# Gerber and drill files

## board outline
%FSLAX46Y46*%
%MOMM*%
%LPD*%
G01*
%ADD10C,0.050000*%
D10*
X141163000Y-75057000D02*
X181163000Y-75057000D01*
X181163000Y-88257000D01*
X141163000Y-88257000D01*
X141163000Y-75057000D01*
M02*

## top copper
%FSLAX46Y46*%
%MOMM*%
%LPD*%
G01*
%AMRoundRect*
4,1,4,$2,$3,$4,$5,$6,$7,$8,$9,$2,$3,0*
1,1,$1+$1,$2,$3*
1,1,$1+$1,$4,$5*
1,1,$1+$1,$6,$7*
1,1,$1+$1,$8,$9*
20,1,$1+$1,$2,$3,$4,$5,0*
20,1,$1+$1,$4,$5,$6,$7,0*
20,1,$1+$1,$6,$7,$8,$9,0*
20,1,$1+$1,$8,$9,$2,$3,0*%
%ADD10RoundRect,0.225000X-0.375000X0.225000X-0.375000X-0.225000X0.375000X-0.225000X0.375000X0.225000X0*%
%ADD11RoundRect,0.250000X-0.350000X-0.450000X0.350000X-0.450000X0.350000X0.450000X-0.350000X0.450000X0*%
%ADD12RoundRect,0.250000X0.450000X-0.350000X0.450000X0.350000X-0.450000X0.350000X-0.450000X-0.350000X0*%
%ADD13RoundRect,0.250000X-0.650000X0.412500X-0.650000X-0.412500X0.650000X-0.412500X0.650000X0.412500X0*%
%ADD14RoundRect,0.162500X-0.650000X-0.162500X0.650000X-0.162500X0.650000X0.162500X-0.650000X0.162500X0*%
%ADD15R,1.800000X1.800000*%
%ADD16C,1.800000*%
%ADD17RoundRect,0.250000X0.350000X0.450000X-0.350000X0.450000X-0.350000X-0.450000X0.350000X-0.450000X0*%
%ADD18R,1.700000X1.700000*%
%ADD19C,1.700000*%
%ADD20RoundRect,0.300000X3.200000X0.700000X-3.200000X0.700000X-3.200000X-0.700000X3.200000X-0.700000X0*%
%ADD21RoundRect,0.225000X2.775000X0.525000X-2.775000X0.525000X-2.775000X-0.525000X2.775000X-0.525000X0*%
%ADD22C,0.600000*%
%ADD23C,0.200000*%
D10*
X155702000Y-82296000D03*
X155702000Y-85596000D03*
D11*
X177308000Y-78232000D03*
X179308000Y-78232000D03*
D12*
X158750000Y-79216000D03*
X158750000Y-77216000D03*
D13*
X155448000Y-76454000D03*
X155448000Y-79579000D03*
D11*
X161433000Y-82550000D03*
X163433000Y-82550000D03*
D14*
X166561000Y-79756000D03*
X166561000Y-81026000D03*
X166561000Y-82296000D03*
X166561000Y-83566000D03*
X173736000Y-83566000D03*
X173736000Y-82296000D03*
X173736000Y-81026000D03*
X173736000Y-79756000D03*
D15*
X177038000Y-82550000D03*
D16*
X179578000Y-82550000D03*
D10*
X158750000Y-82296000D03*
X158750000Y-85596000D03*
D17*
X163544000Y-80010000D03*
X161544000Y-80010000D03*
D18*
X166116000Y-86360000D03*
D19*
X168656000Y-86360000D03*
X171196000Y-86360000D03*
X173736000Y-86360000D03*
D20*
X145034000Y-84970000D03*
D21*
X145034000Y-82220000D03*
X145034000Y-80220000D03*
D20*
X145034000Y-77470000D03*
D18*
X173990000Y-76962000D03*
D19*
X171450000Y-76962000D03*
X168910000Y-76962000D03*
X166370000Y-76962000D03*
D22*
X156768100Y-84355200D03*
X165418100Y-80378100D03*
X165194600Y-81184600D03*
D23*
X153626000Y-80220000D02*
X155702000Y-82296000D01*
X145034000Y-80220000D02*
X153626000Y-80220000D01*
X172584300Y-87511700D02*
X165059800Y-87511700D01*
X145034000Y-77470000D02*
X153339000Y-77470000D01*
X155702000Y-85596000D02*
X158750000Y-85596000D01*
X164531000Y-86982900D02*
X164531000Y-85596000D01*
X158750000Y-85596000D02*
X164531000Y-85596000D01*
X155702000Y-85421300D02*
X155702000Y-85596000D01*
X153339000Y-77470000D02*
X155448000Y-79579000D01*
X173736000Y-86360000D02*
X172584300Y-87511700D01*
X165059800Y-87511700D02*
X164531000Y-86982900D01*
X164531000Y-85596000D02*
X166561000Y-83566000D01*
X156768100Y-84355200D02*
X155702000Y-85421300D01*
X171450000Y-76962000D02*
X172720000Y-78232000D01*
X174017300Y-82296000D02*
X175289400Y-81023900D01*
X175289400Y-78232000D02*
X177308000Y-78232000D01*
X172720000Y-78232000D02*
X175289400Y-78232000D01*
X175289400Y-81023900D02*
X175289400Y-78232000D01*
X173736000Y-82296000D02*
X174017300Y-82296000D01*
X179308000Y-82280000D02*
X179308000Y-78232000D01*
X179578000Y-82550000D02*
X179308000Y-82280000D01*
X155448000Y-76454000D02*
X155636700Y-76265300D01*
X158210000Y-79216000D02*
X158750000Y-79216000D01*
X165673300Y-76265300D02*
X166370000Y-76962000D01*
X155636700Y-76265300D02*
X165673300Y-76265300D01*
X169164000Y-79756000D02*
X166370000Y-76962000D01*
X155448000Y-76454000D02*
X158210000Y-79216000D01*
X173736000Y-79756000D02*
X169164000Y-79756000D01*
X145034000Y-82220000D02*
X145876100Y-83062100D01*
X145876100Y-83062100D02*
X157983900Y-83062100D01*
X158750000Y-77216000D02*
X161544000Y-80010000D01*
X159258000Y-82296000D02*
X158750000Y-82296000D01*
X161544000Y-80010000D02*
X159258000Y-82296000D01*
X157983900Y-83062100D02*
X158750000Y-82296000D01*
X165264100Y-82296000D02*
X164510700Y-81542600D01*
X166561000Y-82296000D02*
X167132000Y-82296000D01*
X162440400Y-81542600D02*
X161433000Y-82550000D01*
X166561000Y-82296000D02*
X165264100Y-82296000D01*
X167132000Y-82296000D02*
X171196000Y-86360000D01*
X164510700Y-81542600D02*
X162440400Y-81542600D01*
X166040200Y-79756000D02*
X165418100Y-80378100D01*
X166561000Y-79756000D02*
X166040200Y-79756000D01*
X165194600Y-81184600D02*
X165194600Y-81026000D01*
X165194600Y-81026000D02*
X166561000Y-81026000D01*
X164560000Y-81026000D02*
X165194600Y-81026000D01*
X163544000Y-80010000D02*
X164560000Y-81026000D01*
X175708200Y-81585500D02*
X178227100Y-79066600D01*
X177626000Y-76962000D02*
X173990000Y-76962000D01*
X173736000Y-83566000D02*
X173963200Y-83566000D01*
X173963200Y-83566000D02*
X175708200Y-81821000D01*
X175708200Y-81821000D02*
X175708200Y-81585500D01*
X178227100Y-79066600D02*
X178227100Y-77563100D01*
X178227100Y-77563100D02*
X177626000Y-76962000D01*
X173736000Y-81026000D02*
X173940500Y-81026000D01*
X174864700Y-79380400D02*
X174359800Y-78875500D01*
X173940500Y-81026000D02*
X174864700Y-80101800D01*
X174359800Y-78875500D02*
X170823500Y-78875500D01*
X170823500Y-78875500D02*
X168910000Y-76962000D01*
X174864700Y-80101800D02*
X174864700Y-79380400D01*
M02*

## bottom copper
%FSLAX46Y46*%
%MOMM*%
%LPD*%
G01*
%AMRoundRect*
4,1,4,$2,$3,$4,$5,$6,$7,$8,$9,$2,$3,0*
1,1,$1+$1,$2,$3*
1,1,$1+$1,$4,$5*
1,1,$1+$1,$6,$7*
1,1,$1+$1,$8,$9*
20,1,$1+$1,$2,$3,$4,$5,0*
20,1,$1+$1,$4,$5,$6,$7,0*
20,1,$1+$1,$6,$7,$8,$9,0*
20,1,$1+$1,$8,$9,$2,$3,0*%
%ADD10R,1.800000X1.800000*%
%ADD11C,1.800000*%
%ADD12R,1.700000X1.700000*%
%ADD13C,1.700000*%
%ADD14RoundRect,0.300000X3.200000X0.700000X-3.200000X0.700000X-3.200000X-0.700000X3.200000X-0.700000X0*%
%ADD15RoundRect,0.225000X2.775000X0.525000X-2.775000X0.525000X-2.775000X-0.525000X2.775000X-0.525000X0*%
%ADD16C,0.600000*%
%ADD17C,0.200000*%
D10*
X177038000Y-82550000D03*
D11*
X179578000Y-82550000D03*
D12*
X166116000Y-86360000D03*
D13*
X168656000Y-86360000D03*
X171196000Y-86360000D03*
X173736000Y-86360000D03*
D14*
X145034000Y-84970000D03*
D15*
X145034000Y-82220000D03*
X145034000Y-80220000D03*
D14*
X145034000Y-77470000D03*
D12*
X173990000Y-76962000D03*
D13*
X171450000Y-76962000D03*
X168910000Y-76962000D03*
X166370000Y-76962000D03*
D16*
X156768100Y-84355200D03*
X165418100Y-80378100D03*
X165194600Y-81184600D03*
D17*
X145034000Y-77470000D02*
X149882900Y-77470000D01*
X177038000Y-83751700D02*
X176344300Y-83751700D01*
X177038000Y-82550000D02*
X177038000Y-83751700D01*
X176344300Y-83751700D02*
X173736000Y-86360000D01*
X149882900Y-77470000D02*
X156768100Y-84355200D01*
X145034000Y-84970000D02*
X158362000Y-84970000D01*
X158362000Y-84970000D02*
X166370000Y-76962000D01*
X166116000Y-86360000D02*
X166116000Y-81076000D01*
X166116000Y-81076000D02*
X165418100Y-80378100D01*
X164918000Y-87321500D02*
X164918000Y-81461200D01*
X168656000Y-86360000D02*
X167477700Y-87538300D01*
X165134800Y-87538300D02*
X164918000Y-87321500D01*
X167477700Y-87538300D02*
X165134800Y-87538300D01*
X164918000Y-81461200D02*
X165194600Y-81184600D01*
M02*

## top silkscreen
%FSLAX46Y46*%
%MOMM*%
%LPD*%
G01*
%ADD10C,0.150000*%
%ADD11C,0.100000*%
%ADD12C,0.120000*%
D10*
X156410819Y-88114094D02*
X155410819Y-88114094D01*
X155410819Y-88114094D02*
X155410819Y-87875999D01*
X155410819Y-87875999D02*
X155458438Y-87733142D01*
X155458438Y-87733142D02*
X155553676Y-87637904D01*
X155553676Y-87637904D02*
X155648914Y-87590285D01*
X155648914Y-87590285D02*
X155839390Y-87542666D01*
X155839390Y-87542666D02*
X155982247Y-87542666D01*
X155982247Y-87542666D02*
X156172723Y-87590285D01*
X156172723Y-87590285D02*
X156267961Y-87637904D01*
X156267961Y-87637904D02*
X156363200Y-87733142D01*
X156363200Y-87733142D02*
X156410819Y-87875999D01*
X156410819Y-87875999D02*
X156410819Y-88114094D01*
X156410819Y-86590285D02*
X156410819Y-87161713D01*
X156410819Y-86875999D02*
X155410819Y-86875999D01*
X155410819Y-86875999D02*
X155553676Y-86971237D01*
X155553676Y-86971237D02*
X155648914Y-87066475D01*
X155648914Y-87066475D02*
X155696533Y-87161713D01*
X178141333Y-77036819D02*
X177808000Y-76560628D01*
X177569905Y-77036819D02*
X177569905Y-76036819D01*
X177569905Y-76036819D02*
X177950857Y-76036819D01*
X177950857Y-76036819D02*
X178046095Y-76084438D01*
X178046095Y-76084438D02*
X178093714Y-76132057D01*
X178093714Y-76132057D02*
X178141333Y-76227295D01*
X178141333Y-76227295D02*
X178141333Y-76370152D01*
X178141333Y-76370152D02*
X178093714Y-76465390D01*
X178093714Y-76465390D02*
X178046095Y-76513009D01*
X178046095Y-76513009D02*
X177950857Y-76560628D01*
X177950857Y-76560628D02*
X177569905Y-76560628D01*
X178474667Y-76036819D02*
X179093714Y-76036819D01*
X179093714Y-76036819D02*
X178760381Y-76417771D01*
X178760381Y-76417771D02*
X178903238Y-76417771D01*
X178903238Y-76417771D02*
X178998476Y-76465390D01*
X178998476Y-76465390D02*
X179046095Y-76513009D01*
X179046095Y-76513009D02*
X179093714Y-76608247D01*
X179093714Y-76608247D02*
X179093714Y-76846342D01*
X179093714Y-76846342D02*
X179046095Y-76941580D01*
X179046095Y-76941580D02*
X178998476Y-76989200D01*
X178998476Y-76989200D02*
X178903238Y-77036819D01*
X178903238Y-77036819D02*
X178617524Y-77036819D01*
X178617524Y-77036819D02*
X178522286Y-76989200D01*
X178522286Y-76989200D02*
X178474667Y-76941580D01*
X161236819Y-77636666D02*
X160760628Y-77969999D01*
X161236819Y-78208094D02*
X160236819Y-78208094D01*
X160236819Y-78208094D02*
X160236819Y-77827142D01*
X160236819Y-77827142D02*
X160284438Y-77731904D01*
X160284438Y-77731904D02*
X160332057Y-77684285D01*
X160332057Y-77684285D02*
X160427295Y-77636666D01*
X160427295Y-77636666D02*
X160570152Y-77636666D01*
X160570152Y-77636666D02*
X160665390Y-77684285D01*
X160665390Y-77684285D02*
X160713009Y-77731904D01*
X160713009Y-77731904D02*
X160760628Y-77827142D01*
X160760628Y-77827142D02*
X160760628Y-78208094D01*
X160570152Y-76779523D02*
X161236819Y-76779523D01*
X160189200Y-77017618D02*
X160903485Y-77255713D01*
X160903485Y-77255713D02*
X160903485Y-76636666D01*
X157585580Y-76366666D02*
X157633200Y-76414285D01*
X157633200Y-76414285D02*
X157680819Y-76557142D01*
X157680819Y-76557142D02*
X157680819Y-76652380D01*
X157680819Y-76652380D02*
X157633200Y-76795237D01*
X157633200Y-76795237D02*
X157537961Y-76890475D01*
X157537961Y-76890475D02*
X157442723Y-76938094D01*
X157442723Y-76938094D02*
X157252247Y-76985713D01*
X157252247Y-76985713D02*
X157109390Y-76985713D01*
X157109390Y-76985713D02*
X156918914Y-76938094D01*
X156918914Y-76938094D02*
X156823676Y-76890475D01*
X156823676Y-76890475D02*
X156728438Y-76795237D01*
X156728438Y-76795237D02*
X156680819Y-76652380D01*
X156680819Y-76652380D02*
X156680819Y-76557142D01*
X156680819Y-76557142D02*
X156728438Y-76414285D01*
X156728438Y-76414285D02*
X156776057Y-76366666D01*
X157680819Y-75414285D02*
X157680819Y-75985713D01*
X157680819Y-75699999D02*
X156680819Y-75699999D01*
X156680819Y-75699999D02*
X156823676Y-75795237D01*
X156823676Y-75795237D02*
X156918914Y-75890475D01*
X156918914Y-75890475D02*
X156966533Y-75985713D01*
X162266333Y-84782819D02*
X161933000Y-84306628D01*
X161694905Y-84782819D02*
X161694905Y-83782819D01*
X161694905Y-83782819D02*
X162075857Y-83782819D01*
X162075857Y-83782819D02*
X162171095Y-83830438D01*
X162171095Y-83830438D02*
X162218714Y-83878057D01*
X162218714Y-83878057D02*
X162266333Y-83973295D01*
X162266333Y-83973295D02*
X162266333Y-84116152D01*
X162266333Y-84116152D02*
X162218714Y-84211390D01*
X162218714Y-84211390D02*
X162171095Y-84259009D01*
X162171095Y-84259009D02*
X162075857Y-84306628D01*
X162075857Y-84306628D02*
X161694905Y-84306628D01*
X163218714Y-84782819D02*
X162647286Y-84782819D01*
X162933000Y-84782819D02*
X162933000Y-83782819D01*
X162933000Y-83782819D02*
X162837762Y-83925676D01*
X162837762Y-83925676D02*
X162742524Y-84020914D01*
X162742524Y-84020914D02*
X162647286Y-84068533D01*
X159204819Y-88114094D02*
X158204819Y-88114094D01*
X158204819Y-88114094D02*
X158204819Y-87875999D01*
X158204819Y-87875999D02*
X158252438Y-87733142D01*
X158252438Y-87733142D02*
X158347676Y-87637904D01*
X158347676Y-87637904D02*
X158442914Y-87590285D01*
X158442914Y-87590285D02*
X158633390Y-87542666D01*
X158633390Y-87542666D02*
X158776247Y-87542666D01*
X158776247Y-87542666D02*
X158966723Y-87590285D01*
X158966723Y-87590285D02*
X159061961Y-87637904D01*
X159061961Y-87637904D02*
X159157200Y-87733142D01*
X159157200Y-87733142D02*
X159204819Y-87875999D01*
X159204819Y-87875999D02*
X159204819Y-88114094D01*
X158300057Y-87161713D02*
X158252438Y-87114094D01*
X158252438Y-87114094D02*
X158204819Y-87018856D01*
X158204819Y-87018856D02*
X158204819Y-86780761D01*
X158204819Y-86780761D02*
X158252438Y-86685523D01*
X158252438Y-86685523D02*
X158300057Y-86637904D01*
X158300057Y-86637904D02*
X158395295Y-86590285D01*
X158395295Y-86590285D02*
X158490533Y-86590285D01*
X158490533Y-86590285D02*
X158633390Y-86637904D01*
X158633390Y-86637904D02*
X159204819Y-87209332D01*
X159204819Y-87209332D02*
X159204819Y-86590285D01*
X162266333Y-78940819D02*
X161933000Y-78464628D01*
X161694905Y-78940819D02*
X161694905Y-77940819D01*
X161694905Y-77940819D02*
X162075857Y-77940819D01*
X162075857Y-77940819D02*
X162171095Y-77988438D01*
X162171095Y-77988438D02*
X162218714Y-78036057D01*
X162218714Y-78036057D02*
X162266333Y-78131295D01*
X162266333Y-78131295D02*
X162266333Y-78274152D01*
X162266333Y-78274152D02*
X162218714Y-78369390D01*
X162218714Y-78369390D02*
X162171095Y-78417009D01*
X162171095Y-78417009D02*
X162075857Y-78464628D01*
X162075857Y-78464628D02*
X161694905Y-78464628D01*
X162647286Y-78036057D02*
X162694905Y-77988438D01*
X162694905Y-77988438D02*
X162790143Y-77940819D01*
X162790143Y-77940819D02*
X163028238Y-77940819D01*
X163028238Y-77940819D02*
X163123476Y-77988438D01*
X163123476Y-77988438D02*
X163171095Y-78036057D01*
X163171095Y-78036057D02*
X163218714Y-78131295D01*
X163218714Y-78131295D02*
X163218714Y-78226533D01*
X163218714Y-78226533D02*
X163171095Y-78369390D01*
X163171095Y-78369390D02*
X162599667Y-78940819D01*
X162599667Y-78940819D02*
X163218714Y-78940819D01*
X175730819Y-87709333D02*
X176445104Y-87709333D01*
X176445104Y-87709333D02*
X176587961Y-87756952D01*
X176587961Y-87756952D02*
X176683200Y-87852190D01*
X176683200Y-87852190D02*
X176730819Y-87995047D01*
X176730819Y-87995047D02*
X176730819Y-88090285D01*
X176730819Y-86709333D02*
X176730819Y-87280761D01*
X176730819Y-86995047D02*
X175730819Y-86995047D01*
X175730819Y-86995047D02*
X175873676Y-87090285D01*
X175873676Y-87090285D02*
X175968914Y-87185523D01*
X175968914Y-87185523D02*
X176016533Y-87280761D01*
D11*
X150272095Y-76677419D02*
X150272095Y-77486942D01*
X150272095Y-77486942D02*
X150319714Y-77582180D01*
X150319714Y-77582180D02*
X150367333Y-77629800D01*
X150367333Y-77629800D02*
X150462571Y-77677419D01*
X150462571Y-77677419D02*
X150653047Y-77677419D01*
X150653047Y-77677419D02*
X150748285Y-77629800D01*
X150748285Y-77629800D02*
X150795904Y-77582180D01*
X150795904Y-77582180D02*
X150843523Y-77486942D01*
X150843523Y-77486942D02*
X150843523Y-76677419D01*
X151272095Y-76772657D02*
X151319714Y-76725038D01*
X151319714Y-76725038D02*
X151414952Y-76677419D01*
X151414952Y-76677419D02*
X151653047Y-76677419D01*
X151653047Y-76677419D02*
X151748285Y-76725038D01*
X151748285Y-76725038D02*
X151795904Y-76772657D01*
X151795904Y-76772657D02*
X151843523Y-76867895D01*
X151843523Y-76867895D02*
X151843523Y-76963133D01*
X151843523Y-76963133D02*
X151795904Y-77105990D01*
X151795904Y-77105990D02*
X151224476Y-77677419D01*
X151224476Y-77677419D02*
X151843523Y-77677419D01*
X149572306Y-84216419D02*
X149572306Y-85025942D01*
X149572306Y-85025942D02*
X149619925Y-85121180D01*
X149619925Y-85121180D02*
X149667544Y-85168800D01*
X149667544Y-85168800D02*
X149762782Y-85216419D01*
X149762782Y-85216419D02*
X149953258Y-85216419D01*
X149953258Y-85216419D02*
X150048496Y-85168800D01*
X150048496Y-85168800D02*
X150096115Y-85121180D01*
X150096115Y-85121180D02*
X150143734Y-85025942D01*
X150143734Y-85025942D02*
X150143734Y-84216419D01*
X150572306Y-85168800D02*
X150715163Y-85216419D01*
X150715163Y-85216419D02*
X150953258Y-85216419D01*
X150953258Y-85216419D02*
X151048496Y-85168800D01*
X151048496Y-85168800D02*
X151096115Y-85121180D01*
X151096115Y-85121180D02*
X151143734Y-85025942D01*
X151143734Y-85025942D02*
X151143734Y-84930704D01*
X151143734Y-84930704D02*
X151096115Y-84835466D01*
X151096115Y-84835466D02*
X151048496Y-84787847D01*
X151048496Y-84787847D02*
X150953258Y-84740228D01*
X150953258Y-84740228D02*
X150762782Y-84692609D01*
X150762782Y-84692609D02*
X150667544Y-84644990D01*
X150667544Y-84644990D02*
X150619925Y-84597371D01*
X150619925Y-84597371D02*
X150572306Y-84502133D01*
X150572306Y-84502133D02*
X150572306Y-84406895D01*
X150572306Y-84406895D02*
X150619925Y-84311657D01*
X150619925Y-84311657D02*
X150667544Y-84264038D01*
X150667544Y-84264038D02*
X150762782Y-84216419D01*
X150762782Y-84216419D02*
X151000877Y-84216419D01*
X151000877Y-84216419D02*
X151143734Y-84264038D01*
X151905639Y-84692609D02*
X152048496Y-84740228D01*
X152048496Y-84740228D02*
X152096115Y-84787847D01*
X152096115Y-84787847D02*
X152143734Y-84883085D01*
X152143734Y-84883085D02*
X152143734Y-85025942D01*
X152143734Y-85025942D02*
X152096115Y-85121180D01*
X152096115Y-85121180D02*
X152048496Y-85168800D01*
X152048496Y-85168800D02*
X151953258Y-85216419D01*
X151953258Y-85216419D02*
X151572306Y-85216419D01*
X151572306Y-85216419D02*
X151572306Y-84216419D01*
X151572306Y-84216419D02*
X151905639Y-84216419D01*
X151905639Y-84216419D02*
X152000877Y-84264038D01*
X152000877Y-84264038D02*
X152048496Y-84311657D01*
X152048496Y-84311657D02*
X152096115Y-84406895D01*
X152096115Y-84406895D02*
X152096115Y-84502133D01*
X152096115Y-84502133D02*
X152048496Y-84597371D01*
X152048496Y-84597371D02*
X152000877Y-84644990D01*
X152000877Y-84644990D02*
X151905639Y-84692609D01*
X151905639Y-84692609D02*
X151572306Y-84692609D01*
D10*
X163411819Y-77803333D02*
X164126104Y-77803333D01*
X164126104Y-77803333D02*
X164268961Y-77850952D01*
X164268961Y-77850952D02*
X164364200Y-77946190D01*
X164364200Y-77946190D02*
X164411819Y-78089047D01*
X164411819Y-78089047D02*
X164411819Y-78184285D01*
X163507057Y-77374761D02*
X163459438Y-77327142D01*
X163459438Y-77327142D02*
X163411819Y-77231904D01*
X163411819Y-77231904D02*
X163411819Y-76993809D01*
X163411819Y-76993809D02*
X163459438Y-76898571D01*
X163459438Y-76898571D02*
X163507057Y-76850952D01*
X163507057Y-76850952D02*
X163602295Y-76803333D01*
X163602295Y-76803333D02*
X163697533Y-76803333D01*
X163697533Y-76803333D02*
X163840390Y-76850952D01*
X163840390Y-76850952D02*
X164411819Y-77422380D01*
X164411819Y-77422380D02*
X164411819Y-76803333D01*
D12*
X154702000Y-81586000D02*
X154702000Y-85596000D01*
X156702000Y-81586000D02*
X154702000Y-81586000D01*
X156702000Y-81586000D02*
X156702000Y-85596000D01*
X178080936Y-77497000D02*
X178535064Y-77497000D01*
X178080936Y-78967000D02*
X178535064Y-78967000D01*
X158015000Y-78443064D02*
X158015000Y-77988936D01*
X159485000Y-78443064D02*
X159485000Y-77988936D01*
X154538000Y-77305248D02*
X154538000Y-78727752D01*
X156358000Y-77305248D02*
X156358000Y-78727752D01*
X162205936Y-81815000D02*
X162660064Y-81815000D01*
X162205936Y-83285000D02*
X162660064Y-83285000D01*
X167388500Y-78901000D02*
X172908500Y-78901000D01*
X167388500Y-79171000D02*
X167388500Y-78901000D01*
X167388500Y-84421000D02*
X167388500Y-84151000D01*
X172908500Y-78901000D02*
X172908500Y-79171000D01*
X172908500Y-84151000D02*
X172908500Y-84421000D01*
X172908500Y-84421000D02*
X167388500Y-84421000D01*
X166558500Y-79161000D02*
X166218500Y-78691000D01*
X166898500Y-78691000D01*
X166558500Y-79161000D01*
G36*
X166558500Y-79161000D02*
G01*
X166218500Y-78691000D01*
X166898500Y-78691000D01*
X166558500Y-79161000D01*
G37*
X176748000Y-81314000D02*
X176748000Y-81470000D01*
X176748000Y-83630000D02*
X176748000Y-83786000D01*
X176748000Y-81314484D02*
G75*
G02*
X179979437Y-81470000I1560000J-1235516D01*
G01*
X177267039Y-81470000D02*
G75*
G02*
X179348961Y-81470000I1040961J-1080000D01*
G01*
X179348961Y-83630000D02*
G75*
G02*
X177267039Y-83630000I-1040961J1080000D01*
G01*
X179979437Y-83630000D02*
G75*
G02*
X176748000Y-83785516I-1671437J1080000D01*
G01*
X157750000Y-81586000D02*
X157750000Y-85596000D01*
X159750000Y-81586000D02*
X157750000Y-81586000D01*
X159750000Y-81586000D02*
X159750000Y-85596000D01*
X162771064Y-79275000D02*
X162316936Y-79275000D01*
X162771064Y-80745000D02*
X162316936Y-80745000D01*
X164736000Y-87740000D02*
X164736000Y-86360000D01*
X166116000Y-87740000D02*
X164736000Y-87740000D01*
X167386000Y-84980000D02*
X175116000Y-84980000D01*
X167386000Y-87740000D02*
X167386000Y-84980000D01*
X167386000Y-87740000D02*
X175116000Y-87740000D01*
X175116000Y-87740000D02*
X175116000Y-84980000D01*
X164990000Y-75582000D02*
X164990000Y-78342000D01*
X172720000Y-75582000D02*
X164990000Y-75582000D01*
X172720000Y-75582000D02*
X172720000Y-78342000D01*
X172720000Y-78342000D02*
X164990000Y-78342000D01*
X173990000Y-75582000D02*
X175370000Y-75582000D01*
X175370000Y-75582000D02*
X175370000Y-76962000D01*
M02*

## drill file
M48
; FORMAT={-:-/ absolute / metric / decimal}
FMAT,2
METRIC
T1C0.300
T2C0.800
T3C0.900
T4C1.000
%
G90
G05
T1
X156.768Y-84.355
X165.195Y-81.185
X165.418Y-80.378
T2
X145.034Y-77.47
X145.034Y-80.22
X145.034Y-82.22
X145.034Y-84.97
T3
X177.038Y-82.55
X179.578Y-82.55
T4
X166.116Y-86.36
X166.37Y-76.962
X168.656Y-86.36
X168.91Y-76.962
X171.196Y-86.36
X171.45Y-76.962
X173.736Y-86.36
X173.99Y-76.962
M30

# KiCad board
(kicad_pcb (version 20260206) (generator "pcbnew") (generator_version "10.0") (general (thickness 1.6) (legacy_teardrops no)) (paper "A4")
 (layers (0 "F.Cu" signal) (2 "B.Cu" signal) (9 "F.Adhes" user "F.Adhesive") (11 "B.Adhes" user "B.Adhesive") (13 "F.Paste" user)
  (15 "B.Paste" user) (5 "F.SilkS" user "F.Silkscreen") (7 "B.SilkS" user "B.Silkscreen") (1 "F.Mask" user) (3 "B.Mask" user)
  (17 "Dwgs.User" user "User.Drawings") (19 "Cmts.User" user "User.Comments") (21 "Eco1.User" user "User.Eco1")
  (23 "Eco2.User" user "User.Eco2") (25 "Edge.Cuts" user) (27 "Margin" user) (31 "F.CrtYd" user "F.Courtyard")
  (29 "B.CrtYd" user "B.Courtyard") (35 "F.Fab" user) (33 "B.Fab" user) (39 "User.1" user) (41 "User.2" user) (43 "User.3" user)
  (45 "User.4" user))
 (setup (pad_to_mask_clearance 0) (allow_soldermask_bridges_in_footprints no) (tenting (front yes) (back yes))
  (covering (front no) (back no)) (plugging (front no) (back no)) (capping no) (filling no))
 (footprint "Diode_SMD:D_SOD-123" (layer "F.Cu") (at 155.702 83.946 -90)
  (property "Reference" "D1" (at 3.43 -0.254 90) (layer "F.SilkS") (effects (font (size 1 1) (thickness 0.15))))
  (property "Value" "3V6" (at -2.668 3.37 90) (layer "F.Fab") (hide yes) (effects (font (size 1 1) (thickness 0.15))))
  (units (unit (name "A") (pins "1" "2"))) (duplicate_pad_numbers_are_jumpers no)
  (fp_line (start -2.36 1) (end 1.65 1) (stroke (width 0.12) (type solid)) (layer "F.SilkS"))
  (fp_line (start -2.36 -1) (end -2.36 1) (stroke (width 0.12) (type solid)) (layer "F.SilkS"))
  (fp_line (start -2.36 -1) (end 1.65 -1) (stroke (width 0.12) (type solid)) (layer "F.SilkS"))
  (pad "1" smd roundrect (at -1.65 0 270) (size 0.9 1.2) (layers "F.Cu" "F.Mask" "F.Paste") (roundrect_rratio 0.25) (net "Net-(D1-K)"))
  (pad "2" smd roundrect (at 1.65 0 270) (size 0.9 1.2) (layers "F.Cu" "F.Mask" "F.Paste") (roundrect_rratio 0.25) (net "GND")))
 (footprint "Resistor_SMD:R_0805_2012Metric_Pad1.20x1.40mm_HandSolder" (layer "F.Cu") (at 178.308 78.232)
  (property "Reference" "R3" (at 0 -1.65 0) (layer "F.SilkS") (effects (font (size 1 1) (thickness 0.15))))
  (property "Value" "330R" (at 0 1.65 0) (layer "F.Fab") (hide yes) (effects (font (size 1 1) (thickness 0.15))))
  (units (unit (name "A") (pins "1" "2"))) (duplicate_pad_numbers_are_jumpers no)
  (fp_line (start -0.227064 -0.735) (end 0.227064 -0.735) (stroke (width 0.12) (type solid)) (layer "F.SilkS"))
  (fp_line (start -0.227064 0.735) (end 0.227064 0.735) (stroke (width 0.12) (type solid)) (layer "F.SilkS"))
  (pad "1" smd roundrect (at -1 0) (size 1.2 1.4) (layers "F.Cu" "F.Mask" "F.Paste") (roundrect_rratio 0.208333) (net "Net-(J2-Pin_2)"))
  (pad "2" smd roundrect (at 1 0) (size 1.2 1.4) (layers "F.Cu" "F.Mask" "F.Paste") (roundrect_rratio 0.208333) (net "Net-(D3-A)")))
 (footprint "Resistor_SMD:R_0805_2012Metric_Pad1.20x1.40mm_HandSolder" (layer "F.Cu") (at 158.75 78.216 90)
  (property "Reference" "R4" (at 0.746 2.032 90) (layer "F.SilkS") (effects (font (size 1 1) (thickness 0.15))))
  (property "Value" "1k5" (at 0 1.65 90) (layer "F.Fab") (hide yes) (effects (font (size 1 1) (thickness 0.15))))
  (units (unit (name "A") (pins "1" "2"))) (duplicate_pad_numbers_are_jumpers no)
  (fp_line (start -0.227064 -0.735) (end 0.227064 -0.735) (stroke (width 0.12) (type solid)) (layer "F.SilkS"))
  (fp_line (start -0.227064 0.735) (end 0.227064 0.735) (stroke (width 0.12) (type solid)) (layer "F.SilkS"))
  (pad "1" smd roundrect (at -1 0 90) (size 1.2 1.4) (layers "F.Cu" "F.Mask" "F.Paste") (roundrect_rratio 0.208333) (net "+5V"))
  (pad "2" smd roundrect (at 1 0 90) (size 1.2 1.4) (layers "F.Cu" "F.Mask" "F.Paste") (roundrect_rratio 0.208333) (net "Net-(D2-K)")))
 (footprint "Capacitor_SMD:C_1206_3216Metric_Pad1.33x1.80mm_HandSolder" (layer "F.Cu") (at 155.448 78.0165 -90)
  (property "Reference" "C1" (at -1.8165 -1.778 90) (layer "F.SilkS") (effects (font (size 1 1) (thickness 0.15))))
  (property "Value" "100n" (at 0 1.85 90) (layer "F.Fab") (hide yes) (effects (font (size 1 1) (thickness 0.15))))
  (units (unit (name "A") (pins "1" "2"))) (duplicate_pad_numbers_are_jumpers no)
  (fp_line (start -0.711252 0.91) (end 0.711252 0.91) (stroke (width 0.12) (type solid)) (layer "F.SilkS"))
  (fp_line (start -0.711252 -0.91) (end 0.711252 -0.91) (stroke (width 0.12) (type solid)) (layer "F.SilkS"))
  (pad "1" smd roundrect (at -1.5625 0 270) (size 1.325 1.8) (layers "F.Cu" "F.Mask" "F.Paste") (roundrect_rratio 0.188679) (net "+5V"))
  (pad "2" smd roundrect (at 1.5625 0 270) (size 1.325 1.8) (layers "F.Cu" "F.Mask" "F.Paste") (roundrect_rratio 0.188679) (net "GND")))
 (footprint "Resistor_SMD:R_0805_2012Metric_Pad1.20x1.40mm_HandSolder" (layer "F.Cu") (at 162.433 82.55)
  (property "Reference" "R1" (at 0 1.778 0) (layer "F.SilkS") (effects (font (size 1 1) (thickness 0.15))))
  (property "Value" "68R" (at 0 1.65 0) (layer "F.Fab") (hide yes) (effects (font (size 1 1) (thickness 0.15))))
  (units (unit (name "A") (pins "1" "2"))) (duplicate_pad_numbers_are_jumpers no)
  (fp_line (start -0.227064 -0.735) (end 0.227064 -0.735) (stroke (width 0.12) (type solid)) (layer "F.SilkS"))
  (fp_line (start -0.227064 0.735) (end 0.227064 0.735) (stroke (width 0.12) (type solid)) (layer "F.SilkS"))
  (pad "1" smd roundrect (at -1 0) (size 1.2 1.4) (layers "F.Cu" "F.Mask" "F.Paste") (roundrect_rratio 0.208333) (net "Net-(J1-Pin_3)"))
  (pad "2" smd roundrect (at 1 0) (size 1.2 1.4) (layers "F.Cu" "F.Mask" "F.Paste") (roundrect_rratio 0.208333) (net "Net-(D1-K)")))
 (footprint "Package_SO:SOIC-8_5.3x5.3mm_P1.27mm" (layer "F.Cu") (at 170.1485 81.661)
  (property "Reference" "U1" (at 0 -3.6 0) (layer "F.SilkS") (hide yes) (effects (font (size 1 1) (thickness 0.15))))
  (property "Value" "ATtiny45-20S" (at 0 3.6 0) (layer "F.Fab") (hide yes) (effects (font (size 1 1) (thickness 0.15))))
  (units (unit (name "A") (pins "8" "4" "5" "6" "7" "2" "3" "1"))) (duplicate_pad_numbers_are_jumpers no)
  (fp_line (start -2.76 -2.76) (end 2.76 -2.76) (stroke (width 0.12) (type solid)) (layer "F.SilkS"))
  (fp_line (start -2.76 -2.49) (end -2.76 -2.76) (stroke (width 0.12) (type solid)) (layer "F.SilkS"))
  (fp_line (start -2.76 2.76) (end -2.76 2.49) (stroke (width 0.12) (type solid)) (layer "F.SilkS"))
  (fp_line (start 2.76 -2.76) (end 2.76 -2.49) (stroke (width 0.12) (type solid)) (layer "F.SilkS"))
  (fp_line (start 2.76 2.49) (end 2.76 2.76) (stroke (width 0.12) (type solid)) (layer "F.SilkS"))
  (fp_line (start 2.76 2.76) (end -2.76 2.76) (stroke (width 0.12) (type solid)) (layer "F.SilkS"))
  (fp_poly (pts (xy -3.59 -2.5) (xy -3.93 -2.97) (xy -3.25 -2.97)) (stroke (width 0.12) (type solid)) (fill yes) (layer "F.SilkS"))
  (pad "1" smd roundrect (at -3.5875 -1.905) (size 1.625 0.65) (layers "F.Cu" "F.Mask" "F.Paste") (roundrect_rratio 0.25)
   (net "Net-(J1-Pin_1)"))
  (pad "2" smd roundrect (at -3.5875 -0.635) (size 1.625 0.65) (layers "F.Cu" "F.Mask" "F.Paste") (roundrect_rratio 0.25)
   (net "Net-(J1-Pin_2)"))
  (pad "3" smd roundrect (at -3.5875 0.635) (size 1.625 0.65) (layers "F.Cu" "F.Mask" "F.Paste") (roundrect_rratio 0.25)
   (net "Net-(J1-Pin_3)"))
  (pad "4" smd roundrect (at -3.5875 1.905) (size 1.625 0.65) (layers "F.Cu" "F.Mask" "F.Paste") (roundrect_rratio 0.25) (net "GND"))
  (pad "5" smd roundrect (at 3.5875 1.905) (size 1.625 0.65) (layers "F.Cu" "F.Mask" "F.Paste") (roundrect_rratio 0.25)
   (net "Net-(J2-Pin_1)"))
  (pad "6" smd roundrect (at 3.5875 0.635) (size 1.625 0.65) (layers "F.Cu" "F.Mask" "F.Paste") (roundrect_rratio 0.25)
   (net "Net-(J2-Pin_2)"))
  (pad "7" smd roundrect (at 3.5875 -0.635) (size 1.625 0.65) (layers "F.Cu" "F.Mask" "F.Paste") (roundrect_rratio 0.25)
   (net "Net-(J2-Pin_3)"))
  (pad "8" smd roundrect (at 3.5875 -1.905) (size 1.625 0.65) (layers "F.Cu" "F.Mask" "F.Paste") (roundrect_rratio 0.25) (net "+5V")))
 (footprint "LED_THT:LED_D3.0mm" (layer "F.Cu") (at 177.038 82.55)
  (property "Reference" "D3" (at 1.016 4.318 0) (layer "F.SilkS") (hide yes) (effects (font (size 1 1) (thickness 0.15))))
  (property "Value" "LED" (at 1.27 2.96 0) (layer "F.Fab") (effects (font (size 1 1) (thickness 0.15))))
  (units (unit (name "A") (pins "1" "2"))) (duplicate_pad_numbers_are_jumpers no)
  (fp_line (start -0.29 -1.236) (end -0.29 -1.08) (stroke (width 0.12) (type solid)) (layer "F.SilkS"))
  (fp_line (start -0.29 1.08) (end -0.29 1.236) (stroke (width 0.12) (type solid)) (layer "F.SilkS"))
  (fp_arc (start -0.29 -1.235516) (mid 1.36566 -1.987699) (end 2.941437 -1.08) (stroke (width 0.12) (type solid)) (layer "F.SilkS"))
  (fp_arc (start 0.229039 -1.08) (mid 1.27 -1.5) (end 2.310961 -1.08) (stroke (width 0.12) (type solid)) (layer "F.SilkS"))
  (fp_arc (start 2.310961 1.08) (mid 1.27 1.5) (end 0.229039 1.08) (stroke (width 0.12) (type solid)) (layer "F.SilkS"))
  (fp_arc (start 2.941437 1.08) (mid 1.36566 1.987699) (end -0.29 1.235516) (stroke (width 0.12) (type solid)) (layer "F.SilkS"))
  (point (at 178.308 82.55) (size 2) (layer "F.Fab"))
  (pad "1" thru_hole rect (at 0 0) (size 1.8 1.8) (drill 0.9) (layers "*.Cu" "*.Mask") (remove_unused_layers no) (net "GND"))
  (pad "2" thru_hole circle (at 2.54 0) (size 1.8 1.8) (drill 0.9) (layers "*.Cu" "*.Mask") (remove_unused_layers no) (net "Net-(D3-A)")))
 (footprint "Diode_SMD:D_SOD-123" (layer "F.Cu") (at 158.75 83.946 -90)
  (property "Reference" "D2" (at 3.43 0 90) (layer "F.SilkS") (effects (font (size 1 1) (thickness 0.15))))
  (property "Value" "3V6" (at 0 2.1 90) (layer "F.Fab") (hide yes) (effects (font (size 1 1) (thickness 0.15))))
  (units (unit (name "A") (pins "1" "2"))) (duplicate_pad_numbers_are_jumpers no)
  (fp_line (start -2.36 1) (end 1.65 1) (stroke (width 0.12) (type solid)) (layer "F.SilkS"))
  (fp_line (start -2.36 -1) (end -2.36 1) (stroke (width 0.12) (type solid)) (layer "F.SilkS"))
  (fp_line (start -2.36 -1) (end 1.65 -1) (stroke (width 0.12) (type solid)) (layer "F.SilkS"))
  (pad "1" smd roundrect (at -1.65 0 270) (size 0.9 1.2) (layers "F.Cu" "F.Mask" "F.Paste") (roundrect_rratio 0.25) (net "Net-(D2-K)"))
  (pad "2" smd roundrect (at 1.65 0 270) (size 0.9 1.2) (layers "F.Cu" "F.Mask" "F.Paste") (roundrect_rratio 0.25) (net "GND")))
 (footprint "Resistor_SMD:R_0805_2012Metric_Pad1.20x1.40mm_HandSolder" (layer "F.Cu") (at 162.544 80.01 180)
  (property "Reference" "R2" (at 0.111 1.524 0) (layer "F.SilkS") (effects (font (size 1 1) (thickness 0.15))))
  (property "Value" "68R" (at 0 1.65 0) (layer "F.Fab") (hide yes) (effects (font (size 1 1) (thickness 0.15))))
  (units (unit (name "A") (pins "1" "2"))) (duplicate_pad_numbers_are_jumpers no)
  (fp_line (start -0.227064 0.735) (end 0.227064 0.735) (stroke (width 0.12) (type solid)) (layer "F.SilkS"))
  (fp_line (start -0.227064 -0.735) (end 0.227064 -0.735) (stroke (width 0.12) (type solid)) (layer "F.SilkS"))
  (pad "1" smd roundrect (at -1 0 180) (size 1.2 1.4) (layers "F.Cu" "F.Mask" "F.Paste") (roundrect_rratio 0.208333) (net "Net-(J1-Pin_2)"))
  (pad "2" smd roundrect (at 1 0 180) (size 1.2 1.4) (layers "F.Cu" "F.Mask" "F.Paste") (roundrect_rratio 0.208333) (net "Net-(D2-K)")))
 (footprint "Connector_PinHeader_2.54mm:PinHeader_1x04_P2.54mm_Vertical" (layer "F.Cu") (at 166.116 86.36 90)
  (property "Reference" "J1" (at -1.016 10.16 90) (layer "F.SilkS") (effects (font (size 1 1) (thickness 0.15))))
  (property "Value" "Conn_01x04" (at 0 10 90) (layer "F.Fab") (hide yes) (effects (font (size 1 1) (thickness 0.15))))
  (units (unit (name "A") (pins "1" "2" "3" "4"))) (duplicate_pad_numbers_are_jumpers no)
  (fp_line (start -1.38 -1.38) (end 0 -1.38) (stroke (width 0.12) (type solid)) (layer "F.SilkS"))
  (fp_line (start -1.38 0) (end -1.38 -1.38) (stroke (width 0.12) (type solid)) (layer "F.SilkS"))
  (fp_line (start 1.38 1.27) (end 1.38 9) (stroke (width 0.12) (type solid)) (layer "F.SilkS"))
  (fp_line (start -1.38 1.27) (end 1.38 1.27) (stroke (width 0.12) (type solid)) (layer "F.SilkS"))
  (fp_line (start -1.38 1.27) (end -1.38 9) (stroke (width 0.12) (type solid)) (layer "F.SilkS"))
  (fp_line (start -1.38 9) (end 1.38 9) (stroke (width 0.12) (type solid)) (layer "F.SilkS"))
  (pad "1" thru_hole rect (at 0 0 90) (size 1.7 1.7) (drill 1) (layers "*.Cu" "*.Mask") (remove_unused_layers no) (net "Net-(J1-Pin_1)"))
  (pad "2" thru_hole circle (at 0 2.54 90) (size 1.7 1.7) (drill 1) (layers "*.Cu" "*.Mask") (remove_unused_layers no)
   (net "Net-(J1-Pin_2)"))
  (pad "3" thru_hole circle (at 0 5.08 90) (size 1.7 1.7) (drill 1) (layers "*.Cu" "*.Mask") (remove_unused_layers no)
   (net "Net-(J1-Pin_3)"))
  (pad "4" thru_hole circle (at 0 7.62 90) (size 1.7 1.7) (drill 1) (layers "*.Cu" "*.Mask") (remove_unused_layers no) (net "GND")))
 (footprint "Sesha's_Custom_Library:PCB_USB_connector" (layer "F.Cu") (at 150.034 81.22 180)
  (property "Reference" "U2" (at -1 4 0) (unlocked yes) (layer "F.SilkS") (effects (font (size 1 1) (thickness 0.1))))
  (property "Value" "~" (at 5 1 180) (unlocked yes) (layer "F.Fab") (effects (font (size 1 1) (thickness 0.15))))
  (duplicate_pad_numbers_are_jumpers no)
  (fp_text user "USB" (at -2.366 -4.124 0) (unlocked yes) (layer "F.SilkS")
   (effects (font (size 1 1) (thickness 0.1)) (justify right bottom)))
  (pad "1" thru_hole roundrect (at 5 -3.75 180) (size 7 2) (drill 0.8) (layers "*.Cu" "*.Mask") (remove_unused_layers no)
   (roundrect_rratio 0.15) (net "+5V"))
  (pad "2" thru_hole roundrect (at 5 -1 180) (size 6 1.5) (drill 0.8) (layers "*.Cu" "*.Mask") (remove_unused_layers no)
   (roundrect_rratio 0.15) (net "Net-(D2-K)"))
  (pad "3" thru_hole roundrect (at 5 1 180) (size 6 1.5) (drill 0.8) (layers "*.Cu" "*.Mask") (remove_unused_layers no)
   (roundrect_rratio 0.15) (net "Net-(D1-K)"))
  (pad "4" thru_hole roundrect (at 5 3.75 180) (size 7 2) (drill 0.8) (layers "*.Cu" "*.Mask") (remove_unused_layers no)
   (roundrect_rratio 0.15) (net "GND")))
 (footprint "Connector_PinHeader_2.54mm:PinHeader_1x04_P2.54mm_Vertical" (layer "F.Cu") (at 173.99 76.962 -90)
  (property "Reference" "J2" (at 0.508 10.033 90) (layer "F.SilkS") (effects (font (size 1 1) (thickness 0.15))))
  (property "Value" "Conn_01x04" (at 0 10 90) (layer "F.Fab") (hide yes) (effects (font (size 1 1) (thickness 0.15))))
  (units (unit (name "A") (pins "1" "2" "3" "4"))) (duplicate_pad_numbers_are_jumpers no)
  (fp_line (start -1.38 9) (end 1.38 9) (stroke (width 0.12) (type solid)) (layer "F.SilkS"))
  (fp_line (start -1.38 1.27) (end -1.38 9) (stroke (width 0.12) (type solid)) (layer "F.SilkS"))
  (fp_line (start -1.38 1.27) (end 1.38 1.27) (stroke (width 0.12) (type solid)) (layer "F.SilkS"))
  (fp_line (start 1.38 1.27) (end 1.38 9) (stroke (width 0.12) (type solid)) (layer "F.SilkS"))
  (fp_line (start -1.38 0) (end -1.38 -1.38) (stroke (width 0.12) (type solid)) (layer "F.SilkS"))
  (fp_line (start -1.38 -1.38) (end 0 -1.38) (stroke (width 0.12) (type solid)) (layer "F.SilkS"))
  (pad "1" thru_hole rect (at 0 0 270) (size 1.7 1.7) (drill 1) (layers "*.Cu" "*.Mask") (remove_unused_layers no) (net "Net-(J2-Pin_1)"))
  (pad "2" thru_hole circle (at 0 2.54 270) (size 1.7 1.7) (drill 1) (layers "*.Cu" "*.Mask") (remove_unused_layers no)
   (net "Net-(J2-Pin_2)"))
  (pad "3" thru_hole circle (at 0 5.08 270) (size 1.7 1.7) (drill 1) (layers "*.Cu" "*.Mask") (remove_unused_layers no)
   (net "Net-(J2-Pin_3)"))
  (pad "4" thru_hole circle (at 0 7.62 270) (size 1.7 1.7) (drill 1) (layers "*.Cu" "*.Mask") (remove_unused_layers no) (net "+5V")))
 (gr_rect (start 141.163 75.057) (end 181.163 88.257) (stroke (width 0.05) (type solid)) (fill no) (layer "Edge.Cuts"))
 (segment (start 153.626 80.22) (end 155.702 82.296) (width 0.2) (layer "F.Cu") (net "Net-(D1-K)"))
 (segment (start 145.034 80.22) (end 153.626 80.22) (width 0.2) (layer "F.Cu") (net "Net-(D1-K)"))
 (segment (start 172.5843 87.5117) (end 165.0598 87.5117) (width 0.2) (layer "F.Cu") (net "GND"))
 (segment (start 145.034 77.47) (end 153.339 77.47) (width 0.2) (layer "F.Cu") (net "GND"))
 (segment (start 155.702 85.596) (end 158.75 85.596) (width 0.2) (layer "F.Cu") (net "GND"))
 (segment (start 164.531 86.9829) (end 164.531 85.596) (width 0.2) (layer "F.Cu") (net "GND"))
 (segment (start 158.75 85.596) (end 164.531 85.596) (width 0.2) (layer "F.Cu") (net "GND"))
 (segment (start 155.702 85.4213) (end 155.702 85.596) (width 0.2) (layer "F.Cu") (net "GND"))
 (segment (start 153.339 77.47) (end 155.448 79.579) (width 0.2) (layer "F.Cu") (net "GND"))
 (segment (start 173.736 86.36) (end 172.5843 87.5117) (width 0.2) (layer "F.Cu") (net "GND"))
 (segment (start 165.0598 87.5117) (end 164.531 86.9829) (width 0.2) (layer "F.Cu") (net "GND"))
 (segment (start 164.531 85.596) (end 166.561 83.566) (width 0.2) (layer "F.Cu") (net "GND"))
 (segment (start 156.7681 84.3552) (end 155.702 85.4213) (width 0.2) (layer "F.Cu") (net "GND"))
 (via (at 156.7681 84.3552) (size 0.6) (drill 0.3) (layers "F.Cu" "B.Cu") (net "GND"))
 (segment (start 145.034 77.47) (end 149.8829 77.47) (width 0.2) (layer "B.Cu") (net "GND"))
 (segment (start 177.038 83.7517) (end 176.3443 83.7517) (width 0.2) (layer "B.Cu") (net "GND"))
 (segment (start 177.038 82.55) (end 177.038 83.7517) (width 0.2) (layer "B.Cu") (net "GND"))
 (segment (start 176.3443 83.7517) (end 173.736 86.36) (width 0.2) (layer "B.Cu") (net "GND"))
 (segment (start 149.8829 77.47) (end 156.7681 84.3552) (width 0.2) (layer "B.Cu") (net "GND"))
 (segment (start 171.45 76.962) (end 172.72 78.232) (width 0.2) (layer "F.Cu") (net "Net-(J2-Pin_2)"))
 (segment (start 174.0173 82.296) (end 175.2894 81.0239) (width 0.2) (layer "F.Cu") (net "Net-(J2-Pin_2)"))
 (segment (start 175.2894 78.232) (end 177.308 78.232) (width 0.2) (layer "F.Cu") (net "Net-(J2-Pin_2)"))
 (segment (start 172.72 78.232) (end 175.2894 78.232) (width 0.2) (layer "F.Cu") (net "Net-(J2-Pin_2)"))
 (segment (start 175.2894 81.0239) (end 175.2894 78.232) (width 0.2) (layer "F.Cu") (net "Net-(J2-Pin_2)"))
 (segment (start 173.736 82.296) (end 174.0173 82.296) (width 0.2) (layer "F.Cu") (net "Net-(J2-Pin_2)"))
 (segment (start 179.308 82.28) (end 179.308 78.232) (width 0.2) (layer "F.Cu") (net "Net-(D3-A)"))
 (segment (start 179.578 82.55) (end 179.308 82.28) (width 0.2) (layer "F.Cu") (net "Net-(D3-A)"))
 (segment (start 155.448 76.454) (end 155.6367 76.2653) (width 0.2) (layer "F.Cu") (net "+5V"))
 (segment (start 158.21 79.216) (end 158.75 79.216) (width 0.2) (layer "F.Cu") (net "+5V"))
 (segment (start 165.6733 76.2653) (end 166.37 76.962) (width 0.2) (layer "F.Cu") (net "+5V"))
 (segment (start 155.6367 76.2653) (end 165.6733 76.2653) (width 0.2) (layer "F.Cu") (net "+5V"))
 (segment (start 169.164 79.756) (end 166.37 76.962) (width 0.2) (layer "F.Cu") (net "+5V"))
 (segment (start 155.448 76.454) (end 158.21 79.216) (width 0.2) (layer "F.Cu") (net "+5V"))
 (segment (start 173.736 79.756) (end 169.164 79.756) (width 0.2) (layer "F.Cu") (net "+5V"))
 (segment (start 145.034 84.97) (end 158.362 84.97) (width 0.2) (layer "B.Cu") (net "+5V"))
 (segment (start 158.362 84.97) (end 166.37 76.962) (width 0.2) (layer "B.Cu") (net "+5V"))
 (segment (start 145.034 82.22) (end 145.8761 83.0621) (width 0.2) (layer "F.Cu") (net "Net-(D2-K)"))
 (segment (start 145.8761 83.0621) (end 157.9839 83.0621) (width 0.2) (layer "F.Cu") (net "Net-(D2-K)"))
 (segment (start 158.75 77.216) (end 161.544 80.01) (width 0.2) (layer "F.Cu") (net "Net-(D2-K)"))
 (segment (start 159.258 82.296) (end 158.75 82.296) (width 0.2) (layer "F.Cu") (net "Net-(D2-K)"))
 (segment (start 161.544 80.01) (end 159.258 82.296) (width 0.2) (layer "F.Cu") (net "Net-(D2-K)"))
 (segment (start 157.9839 83.0621) (end 158.75 82.296) (width 0.2) (layer "F.Cu") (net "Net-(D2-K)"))
 (segment (start 165.2641 82.296) (end 164.5107 81.5426) (width 0.2) (layer "F.Cu") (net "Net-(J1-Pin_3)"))
 (segment (start 166.561 82.296) (end 167.132 82.296) (width 0.2) (layer "F.Cu") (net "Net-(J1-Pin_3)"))
 (segment (start 162.4404 81.5426) (end 161.433 82.55) (width 0.2) (layer "F.Cu") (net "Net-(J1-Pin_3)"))
 (segment (start 166.561 82.296) (end 165.2641 82.296) (width 0.2) (layer "F.Cu") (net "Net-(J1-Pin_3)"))
 (segment (start 167.132 82.296) (end 171.196 86.36) (width 0.2) (layer "F.Cu") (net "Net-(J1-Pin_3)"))
 (segment (start 164.5107 81.5426) (end 162.4404 81.5426) (width 0.2) (layer "F.Cu") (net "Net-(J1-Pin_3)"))
 (segment (start 166.0402 79.756) (end 165.4181 80.3781) (width 0.2) (layer "F.Cu") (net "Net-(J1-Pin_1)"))
 (segment (start 166.561 79.756) (end 166.0402 79.756) (width 0.2) (layer "F.Cu") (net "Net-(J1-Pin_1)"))
 (via (at 165.4181 80.3781) (size 0.6) (drill 0.3) (layers "F.Cu" "B.Cu") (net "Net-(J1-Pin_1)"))
 (segment (start 166.116 86.36) (end 166.116 81.076) (width 0.2) (layer "B.Cu") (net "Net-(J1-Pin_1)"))
 (segment (start 166.116 81.076) (end 165.4181 80.3781) (width 0.2) (layer "B.Cu") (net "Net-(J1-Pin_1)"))
 (segment (start 165.1946 81.1846) (end 165.1946 81.026) (width 0.2) (layer "F.Cu") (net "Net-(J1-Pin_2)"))
 (segment (start 165.1946 81.026) (end 166.561 81.026) (width 0.2) (layer "F.Cu") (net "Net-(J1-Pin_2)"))
 (segment (start 164.56 81.026) (end 165.1946 81.026) (width 0.2) (layer "F.Cu") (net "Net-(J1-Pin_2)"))
 (segment (start 163.544 80.01) (end 164.56 81.026) (width 0.2) (layer "F.Cu") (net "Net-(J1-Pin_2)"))
 (via (at 165.1946 81.1846) (size 0.6) (drill 0.3) (layers "F.Cu" "B.Cu") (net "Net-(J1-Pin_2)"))
 (segment (start 164.918 87.3215) (end 164.918 81.4612) (width 0.2) (layer "B.Cu") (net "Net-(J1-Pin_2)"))
 (segment (start 168.656 86.36) (end 167.4777 87.5383) (width 0.2) (layer "B.Cu") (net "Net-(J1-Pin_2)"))
 (segment (start 165.1348 87.5383) (end 164.918 87.3215) (width 0.2) (layer "B.Cu") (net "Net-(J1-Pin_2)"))
 (segment (start 167.4777 87.5383) (end 165.1348 87.5383) (width 0.2) (layer "B.Cu") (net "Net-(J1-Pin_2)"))
 (segment (start 164.918 81.4612) (end 165.1946 81.1846) (width 0.2) (layer "B.Cu") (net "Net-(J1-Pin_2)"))
 (segment (start 175.7082 81.5855) (end 178.2271 79.0666) (width 0.2) (layer "F.Cu") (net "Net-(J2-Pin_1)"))
 (segment (start 177.626 76.962) (end 173.99 76.962) (width 0.2) (layer "F.Cu") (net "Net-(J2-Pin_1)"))
 (segment (start 173.736 83.566) (end 173.9632 83.566) (width 0.2) (layer "F.Cu") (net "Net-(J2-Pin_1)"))
 (segment (start 173.9632 83.566) (end 175.7082 81.821) (width 0.2) (layer "F.Cu") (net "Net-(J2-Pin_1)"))
 (segment (start 175.7082 81.821) (end 175.7082 81.5855) (width 0.2) (layer "F.Cu") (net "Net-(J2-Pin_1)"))
 (segment (start 178.2271 79.0666) (end 178.2271 77.5631) (width 0.2) (layer "F.Cu") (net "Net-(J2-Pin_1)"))
 (segment (start 178.2271 77.5631) (end 177.626 76.962) (width 0.2) (layer "F.Cu") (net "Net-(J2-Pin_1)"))
 (segment (start 173.736 81.026) (end 173.9405 81.026) (width 0.2) (layer "F.Cu") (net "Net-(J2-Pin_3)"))
 (segment (start 174.8647 79.3804) (end 174.3598 78.8755) (width 0.2) (layer "F.Cu") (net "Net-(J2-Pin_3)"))
 (segment (start 173.9405 81.026) (end 174.8647 80.1018) (width 0.2) (layer "F.Cu") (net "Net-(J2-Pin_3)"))
 (segment (start 174.3598 78.8755) (end 170.8235 78.8755) (width 0.2) (layer "F.Cu") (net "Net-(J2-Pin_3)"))
 (segment (start 170.8235 78.8755) (end 168.91 76.962) (width 0.2) (layer "F.Cu") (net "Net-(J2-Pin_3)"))
 (segment (start 174.8647 80.1018) (end 174.8647 79.3804) (width 0.2) (layer "F.Cu") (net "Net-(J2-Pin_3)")))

